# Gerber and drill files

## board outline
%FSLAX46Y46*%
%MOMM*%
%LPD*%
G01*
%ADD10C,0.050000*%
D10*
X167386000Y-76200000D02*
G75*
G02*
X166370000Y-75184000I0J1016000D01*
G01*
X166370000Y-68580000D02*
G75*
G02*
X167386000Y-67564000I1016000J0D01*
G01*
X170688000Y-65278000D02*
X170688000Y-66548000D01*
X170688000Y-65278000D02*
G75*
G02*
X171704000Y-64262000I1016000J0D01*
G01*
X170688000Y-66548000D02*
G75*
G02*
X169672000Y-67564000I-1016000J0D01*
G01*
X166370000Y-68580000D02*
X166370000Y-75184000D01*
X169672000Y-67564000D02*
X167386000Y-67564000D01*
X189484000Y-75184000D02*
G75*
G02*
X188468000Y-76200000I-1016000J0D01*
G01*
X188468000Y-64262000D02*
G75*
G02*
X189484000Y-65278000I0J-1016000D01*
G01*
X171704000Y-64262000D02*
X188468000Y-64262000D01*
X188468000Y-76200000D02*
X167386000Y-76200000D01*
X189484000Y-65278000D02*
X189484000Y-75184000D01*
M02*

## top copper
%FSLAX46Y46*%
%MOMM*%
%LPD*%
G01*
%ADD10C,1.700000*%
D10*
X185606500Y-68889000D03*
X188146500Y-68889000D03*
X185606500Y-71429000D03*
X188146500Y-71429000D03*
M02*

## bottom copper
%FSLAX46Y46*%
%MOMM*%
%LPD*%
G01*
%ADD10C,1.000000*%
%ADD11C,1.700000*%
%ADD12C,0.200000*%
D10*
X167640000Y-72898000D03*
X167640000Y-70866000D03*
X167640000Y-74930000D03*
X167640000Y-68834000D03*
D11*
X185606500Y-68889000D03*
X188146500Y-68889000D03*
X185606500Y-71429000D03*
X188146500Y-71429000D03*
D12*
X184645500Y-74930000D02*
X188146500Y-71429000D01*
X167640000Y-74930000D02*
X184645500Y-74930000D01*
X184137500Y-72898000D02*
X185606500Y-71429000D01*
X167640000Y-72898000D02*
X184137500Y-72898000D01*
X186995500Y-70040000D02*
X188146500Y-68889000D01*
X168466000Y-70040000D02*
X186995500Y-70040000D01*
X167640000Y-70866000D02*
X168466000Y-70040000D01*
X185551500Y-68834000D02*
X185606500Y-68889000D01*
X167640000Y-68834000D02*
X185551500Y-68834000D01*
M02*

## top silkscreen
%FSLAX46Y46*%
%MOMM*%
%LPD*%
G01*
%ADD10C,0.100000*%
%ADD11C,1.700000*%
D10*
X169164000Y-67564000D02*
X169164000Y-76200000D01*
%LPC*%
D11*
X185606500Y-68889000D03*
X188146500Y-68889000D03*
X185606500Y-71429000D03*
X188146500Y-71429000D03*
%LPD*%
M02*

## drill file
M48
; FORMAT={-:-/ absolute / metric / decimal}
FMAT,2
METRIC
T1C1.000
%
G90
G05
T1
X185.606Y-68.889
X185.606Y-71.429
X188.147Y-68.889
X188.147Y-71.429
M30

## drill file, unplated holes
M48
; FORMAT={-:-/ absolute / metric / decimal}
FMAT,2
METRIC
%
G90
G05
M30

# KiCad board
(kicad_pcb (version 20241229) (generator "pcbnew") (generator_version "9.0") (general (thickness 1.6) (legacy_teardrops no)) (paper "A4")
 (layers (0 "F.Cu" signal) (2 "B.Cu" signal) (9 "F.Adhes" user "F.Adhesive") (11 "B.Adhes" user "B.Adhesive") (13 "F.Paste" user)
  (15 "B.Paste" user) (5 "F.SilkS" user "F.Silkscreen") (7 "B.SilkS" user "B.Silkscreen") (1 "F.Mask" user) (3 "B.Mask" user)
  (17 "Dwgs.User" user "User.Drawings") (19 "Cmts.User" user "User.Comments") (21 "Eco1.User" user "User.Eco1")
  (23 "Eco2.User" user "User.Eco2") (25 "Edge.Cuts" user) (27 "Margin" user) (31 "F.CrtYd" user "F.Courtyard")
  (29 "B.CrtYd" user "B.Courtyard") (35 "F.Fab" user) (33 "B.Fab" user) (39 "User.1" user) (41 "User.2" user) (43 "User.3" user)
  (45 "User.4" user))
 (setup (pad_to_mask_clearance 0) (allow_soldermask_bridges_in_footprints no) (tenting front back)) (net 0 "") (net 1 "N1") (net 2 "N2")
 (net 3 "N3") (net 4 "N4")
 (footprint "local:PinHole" (layer "F.Cu") (at 185.6065 68.889)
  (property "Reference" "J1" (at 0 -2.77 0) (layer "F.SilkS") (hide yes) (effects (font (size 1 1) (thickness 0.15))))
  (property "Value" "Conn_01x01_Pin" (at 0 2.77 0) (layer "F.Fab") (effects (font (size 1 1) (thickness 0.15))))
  (pad "1" thru_hole circle (at 0 0) (size 1.7 1.7) (drill 1) (layers "*.Cu" "*.Mask") (remove_unused_layers no) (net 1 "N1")))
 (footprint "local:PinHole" (layer "F.Cu") (at 188.1465 71.429)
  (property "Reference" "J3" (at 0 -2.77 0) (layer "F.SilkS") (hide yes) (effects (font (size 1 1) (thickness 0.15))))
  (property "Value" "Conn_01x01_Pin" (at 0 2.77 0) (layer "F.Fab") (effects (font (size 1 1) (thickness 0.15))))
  (pad "1" thru_hole circle (at 0 0) (size 1.7 1.7) (drill 1) (layers "*.Cu" "*.Mask") (remove_unused_layers no) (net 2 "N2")))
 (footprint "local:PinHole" (layer "F.Cu") (at 188.1465 68.889)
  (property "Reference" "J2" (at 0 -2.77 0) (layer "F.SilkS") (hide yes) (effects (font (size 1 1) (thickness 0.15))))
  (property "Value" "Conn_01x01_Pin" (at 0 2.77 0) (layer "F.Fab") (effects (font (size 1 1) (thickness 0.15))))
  (pad "1" thru_hole circle (at 0 0) (size 1.7 1.7) (drill 1) (layers "*.Cu" "*.Mask") (remove_unused_layers no) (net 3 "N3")))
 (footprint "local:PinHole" (layer "F.Cu") (at 185.6065 71.429)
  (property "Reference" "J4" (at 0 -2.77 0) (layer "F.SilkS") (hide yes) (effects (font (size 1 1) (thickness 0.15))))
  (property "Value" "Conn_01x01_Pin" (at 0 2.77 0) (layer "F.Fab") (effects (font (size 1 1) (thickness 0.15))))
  (pad "1" thru_hole circle (at 0 0) (size 1.7 1.7) (drill 1) (layers "*.Cu" "*.Mask") (remove_unused_layers no) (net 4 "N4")))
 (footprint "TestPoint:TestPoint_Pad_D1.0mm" (layer "B.Cu") (at 167.64 74.93)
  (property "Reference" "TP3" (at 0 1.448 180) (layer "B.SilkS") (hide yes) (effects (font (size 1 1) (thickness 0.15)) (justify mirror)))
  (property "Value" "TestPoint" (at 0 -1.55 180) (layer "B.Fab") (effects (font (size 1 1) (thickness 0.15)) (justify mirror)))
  (pad "1" smd circle (at 0 0) (size 1 1) (layers "B.Cu" "B.Mask") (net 2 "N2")))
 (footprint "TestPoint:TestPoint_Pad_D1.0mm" (layer "B.Cu") (at 167.64 70.866)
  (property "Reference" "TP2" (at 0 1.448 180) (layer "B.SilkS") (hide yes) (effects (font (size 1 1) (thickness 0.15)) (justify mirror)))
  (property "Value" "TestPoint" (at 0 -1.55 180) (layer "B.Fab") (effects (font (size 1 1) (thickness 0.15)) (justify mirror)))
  (pad "1" smd circle (at 0 0) (size 1 1) (layers "B.Cu" "B.Mask") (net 3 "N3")))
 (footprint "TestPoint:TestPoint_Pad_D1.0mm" (layer "B.Cu") (at 167.64 72.898)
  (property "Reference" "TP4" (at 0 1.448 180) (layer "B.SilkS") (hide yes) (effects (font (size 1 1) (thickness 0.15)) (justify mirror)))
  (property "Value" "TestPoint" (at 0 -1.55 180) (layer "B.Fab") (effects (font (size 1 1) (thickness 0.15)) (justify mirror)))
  (pad "1" smd circle (at 0 0) (size 1 1) (layers "B.Cu" "B.Mask") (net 4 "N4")))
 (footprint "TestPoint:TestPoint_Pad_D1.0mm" (layer "B.Cu") (at 167.64 68.834)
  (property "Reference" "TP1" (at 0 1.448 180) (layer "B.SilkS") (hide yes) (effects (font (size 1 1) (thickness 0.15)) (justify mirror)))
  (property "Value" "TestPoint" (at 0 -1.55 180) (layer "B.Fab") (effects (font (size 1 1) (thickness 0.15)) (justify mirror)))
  (pad "1" smd circle (at 0 0) (size 1 1) (layers "B.Cu" "B.Mask") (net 1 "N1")))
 (gr_line (start 169.164 67.564) (end 169.164 76.2) (stroke (width 0.1) (type default)) (layer "F.SilkS"))
 (gr_line (start 189.484 65.278) (end 189.484 75.184) (stroke (width 0.05) (type default)) (layer "Edge.Cuts"))
 (gr_line (start 169.672 67.564) (end 167.386 67.564) (stroke (width 0.05) (type default)) (layer "Edge.Cuts"))
 (gr_arc (start 170.688 65.278) (mid 170.98558 64.55958) (end 171.704 64.262) (stroke (width 0.05) (type default)) (layer "Edge.Cuts"))
 (gr_line (start 171.704 64.262) (end 188.468 64.262) (stroke (width 0.05) (type default)) (layer "Edge.Cuts"))
 (gr_arc (start 166.37 68.58) (mid 166.66758 67.86158) (end 167.386 67.564) (stroke (width 0.05) (type default)) (layer "Edge.Cuts"))
 (gr_line (start 166.37 68.58) (end 166.37 75.184) (stroke (width 0.05) (type default)) (layer "Edge.Cuts"))
 (gr_arc (start 167.386 76.2) (mid 166.66758 75.90242) (end 166.37 75.184) (stroke (width 0.05) (type default)) (layer "Edge.Cuts"))
 (gr_line (start 188.468 76.2) (end 167.386 76.2) (stroke (width 0.05) (type default)) (layer "Edge.Cuts"))
 (gr_line (start 170.688 65.278) (end 170.688 66.548) (stroke (width 0.05) (type default)) (layer "Edge.Cuts"))
 (gr_arc (start 188.468 64.262) (mid 189.18642 64.55958) (end 189.484 65.278) (stroke (width 0.05) (type default)) (layer "Edge.Cuts"))
 (gr_arc (start 170.688 66.548) (mid 170.39042 67.26642) (end 169.672 67.564) (stroke (width 0.05) (type default)) (layer "Edge.Cuts"))
 (gr_arc (start 189.484 75.184) (mid 189.18642 75.90242) (end 188.468 76.2) (stroke (width 0.05) (type default)) (layer "Edge.Cuts"))
 (segment (start 185.5515 68.834) (end 185.6065 68.889) (width 0.2) (layer "B.Cu") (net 1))
 (segment (start 167.64 68.834) (end 185.5515 68.834) (width 0.2) (layer "B.Cu") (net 1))
 (segment (start 186.9955 70.04) (end 188.1465 68.889) (width 0.2) (layer "B.Cu") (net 3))
 (segment (start 168.466 70.04) (end 186.9955 70.04) (width 0.2) (layer "B.Cu") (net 3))
 (segment (start 167.64 70.866) (end 168.466 70.04) (width 0.2) (layer "B.Cu") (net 3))
 (segment (start 167.64 74.93) (end 184.6455 74.93) (width 0.2) (layer "B.Cu") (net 2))
 (segment (start 184.6455 74.93) (end 188.1465 71.429) (width 0.2) (layer "B.Cu") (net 2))
 (segment (start 167.64 72.898) (end 184.1375 72.898) (width 0.2) (layer "B.Cu") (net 4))
 (segment (start 184.1375 72.898) (end 185.6065 71.429) (width 0.2) (layer "B.Cu") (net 4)))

